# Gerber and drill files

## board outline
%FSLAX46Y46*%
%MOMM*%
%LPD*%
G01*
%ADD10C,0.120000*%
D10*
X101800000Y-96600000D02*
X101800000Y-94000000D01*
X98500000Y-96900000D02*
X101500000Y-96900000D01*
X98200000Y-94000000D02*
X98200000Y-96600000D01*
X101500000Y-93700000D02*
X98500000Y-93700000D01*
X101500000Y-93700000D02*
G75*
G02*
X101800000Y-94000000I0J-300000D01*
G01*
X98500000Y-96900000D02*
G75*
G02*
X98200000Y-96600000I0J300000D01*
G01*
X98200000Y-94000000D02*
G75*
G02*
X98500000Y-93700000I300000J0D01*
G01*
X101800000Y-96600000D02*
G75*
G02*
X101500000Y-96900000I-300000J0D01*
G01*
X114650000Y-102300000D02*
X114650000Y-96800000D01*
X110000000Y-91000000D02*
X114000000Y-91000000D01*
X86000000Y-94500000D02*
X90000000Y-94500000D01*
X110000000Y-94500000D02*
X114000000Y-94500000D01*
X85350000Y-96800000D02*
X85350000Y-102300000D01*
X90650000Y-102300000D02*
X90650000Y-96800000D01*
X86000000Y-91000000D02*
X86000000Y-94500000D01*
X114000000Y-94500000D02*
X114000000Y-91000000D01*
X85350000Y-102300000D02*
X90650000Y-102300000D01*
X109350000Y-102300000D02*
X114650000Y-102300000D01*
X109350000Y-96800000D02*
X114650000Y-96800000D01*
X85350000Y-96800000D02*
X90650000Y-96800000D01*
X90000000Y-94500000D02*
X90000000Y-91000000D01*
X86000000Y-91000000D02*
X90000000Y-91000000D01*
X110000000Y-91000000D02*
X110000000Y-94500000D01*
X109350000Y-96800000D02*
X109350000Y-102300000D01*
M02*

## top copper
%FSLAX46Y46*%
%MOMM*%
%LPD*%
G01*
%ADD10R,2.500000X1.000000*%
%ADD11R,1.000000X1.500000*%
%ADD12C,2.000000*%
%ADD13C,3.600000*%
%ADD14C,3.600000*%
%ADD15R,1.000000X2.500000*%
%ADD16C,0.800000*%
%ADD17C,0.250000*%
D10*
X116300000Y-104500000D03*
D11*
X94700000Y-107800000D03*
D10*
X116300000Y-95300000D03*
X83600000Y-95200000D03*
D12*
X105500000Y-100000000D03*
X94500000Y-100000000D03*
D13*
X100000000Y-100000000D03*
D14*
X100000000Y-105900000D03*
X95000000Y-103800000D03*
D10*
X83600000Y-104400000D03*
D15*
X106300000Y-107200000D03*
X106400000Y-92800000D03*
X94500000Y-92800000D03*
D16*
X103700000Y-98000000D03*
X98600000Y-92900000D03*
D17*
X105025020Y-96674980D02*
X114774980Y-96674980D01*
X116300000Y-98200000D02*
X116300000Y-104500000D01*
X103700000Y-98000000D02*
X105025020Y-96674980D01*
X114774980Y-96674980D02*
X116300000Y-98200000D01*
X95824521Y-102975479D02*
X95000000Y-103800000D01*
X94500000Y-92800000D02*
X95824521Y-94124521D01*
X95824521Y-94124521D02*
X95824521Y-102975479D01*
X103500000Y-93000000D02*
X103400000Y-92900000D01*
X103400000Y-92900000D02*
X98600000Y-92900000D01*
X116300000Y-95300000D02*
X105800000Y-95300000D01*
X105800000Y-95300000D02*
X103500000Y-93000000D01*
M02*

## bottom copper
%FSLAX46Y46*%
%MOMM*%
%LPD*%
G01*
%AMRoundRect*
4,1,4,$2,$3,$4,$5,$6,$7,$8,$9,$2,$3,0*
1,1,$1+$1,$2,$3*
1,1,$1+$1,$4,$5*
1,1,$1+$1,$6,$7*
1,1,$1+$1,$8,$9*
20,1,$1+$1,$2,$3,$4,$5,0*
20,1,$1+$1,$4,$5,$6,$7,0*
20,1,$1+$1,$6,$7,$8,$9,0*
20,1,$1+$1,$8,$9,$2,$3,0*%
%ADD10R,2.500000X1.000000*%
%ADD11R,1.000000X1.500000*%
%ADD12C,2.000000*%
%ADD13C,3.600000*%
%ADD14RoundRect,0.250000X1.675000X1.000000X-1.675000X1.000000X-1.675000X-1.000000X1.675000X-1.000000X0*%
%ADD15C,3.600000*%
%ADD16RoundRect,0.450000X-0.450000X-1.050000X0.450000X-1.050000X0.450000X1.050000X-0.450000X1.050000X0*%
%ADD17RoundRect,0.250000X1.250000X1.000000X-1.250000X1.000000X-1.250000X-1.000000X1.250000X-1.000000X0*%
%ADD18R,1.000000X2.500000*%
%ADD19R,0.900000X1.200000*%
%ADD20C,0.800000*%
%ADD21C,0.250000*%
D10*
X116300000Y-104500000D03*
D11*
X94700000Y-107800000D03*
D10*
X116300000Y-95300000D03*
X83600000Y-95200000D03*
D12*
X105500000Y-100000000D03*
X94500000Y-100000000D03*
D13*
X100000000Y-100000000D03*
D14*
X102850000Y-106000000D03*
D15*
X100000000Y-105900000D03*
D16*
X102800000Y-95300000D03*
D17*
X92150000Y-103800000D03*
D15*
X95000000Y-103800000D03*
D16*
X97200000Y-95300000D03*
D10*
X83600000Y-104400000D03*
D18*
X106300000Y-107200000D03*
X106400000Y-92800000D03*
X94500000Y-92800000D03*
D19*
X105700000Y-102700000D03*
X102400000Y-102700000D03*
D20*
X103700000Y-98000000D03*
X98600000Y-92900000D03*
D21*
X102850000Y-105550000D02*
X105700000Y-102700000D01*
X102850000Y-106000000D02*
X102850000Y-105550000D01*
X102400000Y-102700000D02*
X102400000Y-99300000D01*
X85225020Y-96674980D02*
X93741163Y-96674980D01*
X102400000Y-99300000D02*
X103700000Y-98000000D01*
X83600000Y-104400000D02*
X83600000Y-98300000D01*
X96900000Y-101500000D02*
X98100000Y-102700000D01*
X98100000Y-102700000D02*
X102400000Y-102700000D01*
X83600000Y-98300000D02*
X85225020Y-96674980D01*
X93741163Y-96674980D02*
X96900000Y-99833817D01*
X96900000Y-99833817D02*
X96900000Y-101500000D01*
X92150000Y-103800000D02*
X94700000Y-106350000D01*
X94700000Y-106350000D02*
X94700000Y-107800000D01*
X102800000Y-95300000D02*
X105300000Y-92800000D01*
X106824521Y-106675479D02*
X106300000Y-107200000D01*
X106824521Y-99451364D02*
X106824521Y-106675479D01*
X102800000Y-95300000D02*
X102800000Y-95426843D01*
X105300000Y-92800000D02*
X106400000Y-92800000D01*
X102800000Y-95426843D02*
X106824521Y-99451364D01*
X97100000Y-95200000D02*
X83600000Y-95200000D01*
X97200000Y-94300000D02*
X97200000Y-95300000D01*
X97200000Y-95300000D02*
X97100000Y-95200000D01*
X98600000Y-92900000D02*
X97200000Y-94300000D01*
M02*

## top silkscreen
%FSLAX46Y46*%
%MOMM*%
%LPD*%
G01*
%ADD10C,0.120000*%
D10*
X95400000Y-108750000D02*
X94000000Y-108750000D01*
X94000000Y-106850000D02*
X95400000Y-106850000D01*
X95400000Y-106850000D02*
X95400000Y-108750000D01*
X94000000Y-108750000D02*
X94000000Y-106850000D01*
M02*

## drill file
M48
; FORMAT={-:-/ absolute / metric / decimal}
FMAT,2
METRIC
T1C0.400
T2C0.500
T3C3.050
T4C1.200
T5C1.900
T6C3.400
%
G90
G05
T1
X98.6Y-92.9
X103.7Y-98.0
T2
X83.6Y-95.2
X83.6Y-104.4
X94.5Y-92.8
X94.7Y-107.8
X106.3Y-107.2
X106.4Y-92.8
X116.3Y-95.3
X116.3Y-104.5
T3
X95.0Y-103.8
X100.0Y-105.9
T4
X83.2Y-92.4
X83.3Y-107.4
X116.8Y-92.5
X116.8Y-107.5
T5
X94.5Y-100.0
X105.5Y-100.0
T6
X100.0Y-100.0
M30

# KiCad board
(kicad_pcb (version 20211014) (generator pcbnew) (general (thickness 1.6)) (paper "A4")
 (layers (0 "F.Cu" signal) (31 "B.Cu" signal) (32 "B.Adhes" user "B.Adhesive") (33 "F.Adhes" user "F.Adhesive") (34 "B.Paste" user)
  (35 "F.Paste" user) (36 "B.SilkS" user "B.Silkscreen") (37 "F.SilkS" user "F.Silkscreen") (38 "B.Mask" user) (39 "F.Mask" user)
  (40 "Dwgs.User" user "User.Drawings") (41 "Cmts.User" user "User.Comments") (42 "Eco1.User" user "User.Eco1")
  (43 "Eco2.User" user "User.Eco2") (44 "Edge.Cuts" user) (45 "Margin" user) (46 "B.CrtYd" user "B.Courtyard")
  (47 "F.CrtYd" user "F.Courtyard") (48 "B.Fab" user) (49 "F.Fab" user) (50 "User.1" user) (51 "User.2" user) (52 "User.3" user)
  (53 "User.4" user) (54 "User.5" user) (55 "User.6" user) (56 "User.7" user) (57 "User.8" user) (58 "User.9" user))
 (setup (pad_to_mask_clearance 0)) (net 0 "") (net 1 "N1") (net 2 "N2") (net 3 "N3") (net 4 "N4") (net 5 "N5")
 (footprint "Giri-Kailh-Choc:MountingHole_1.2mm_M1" (layer "F.Cu") (at 116.8 92.5)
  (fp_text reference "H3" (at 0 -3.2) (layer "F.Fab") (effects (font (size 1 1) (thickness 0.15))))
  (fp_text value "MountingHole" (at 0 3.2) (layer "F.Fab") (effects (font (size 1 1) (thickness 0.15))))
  (pad "" np_thru_hole circle (at 0 0) (size 1.2 1.2) (drill 1.2) (layers F&B.Cu *.Mask)))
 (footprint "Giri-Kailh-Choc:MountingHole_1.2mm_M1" (layer "F.Cu") (at 116.8 107.5)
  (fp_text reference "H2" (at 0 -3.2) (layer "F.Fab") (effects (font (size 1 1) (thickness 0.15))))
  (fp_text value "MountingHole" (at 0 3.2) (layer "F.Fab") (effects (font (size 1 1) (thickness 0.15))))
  (pad "" np_thru_hole circle (at 0 0) (size 1.2 1.2) (drill 1.2) (layers F&B.Cu *.Mask)))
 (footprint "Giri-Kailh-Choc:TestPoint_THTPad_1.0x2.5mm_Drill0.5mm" (layer "F.Cu") (at 116.3 104.5)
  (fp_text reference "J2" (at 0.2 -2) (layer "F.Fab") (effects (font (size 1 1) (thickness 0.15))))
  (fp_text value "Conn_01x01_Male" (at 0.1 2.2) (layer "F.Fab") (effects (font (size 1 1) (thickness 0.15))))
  (pad "1" thru_hole rect (at 0 0) (size 2.5 1) (drill 0.5) (layers *.Cu *.Mask) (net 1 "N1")))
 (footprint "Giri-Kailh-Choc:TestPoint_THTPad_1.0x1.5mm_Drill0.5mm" (layer "F.Cu") (at 94.7 107.8 90)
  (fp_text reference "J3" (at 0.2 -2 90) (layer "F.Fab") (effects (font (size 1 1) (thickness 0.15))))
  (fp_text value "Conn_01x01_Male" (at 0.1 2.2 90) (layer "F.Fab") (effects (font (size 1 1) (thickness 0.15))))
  (fp_line (start -0.95 0.7) (end -0.95 -0.7) (layer "F.SilkS") (width 0.12))
  (fp_line (start 0.95 -0.7) (end 0.95 0.7) (layer "F.SilkS") (width 0.12))
  (fp_line (start 0.95 0.7) (end -0.95 0.7) (layer "F.SilkS") (width 0.12))
  (fp_line (start -0.95 -0.7) (end 0.95 -0.7) (layer "F.SilkS") (width 0.12))
  (pad "1" thru_hole rect (at 0 0 90) (size 1.5 1) (drill 0.5) (layers *.Cu *.Mask) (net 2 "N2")))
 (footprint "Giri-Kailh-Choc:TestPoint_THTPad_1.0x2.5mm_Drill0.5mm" (layer "F.Cu") (at 116.3 95.3)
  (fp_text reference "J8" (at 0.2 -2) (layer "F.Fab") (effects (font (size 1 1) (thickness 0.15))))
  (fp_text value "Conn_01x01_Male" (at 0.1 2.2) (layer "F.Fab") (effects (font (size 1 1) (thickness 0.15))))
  (pad "1" thru_hole rect (at 0 0) (size 2.5 1) (drill 0.5) (layers *.Cu *.Mask) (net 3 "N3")))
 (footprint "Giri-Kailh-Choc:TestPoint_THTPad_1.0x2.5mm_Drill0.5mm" (layer "F.Cu") (at 83.6 95.2)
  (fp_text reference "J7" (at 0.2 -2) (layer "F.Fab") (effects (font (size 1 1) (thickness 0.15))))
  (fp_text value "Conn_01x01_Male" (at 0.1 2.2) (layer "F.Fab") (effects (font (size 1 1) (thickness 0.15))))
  (pad "1" thru_hole rect (at 0 0) (size 2.5 1) (drill 0.5) (layers *.Cu *.Mask) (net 3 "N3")))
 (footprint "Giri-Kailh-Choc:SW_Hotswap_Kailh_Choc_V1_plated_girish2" (layer "F.Cu") (at 100 100)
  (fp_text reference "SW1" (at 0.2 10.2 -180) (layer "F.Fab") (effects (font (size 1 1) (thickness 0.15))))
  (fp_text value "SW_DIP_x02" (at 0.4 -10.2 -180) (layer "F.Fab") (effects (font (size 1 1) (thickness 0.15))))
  (fp_line (start 1.8 -3.4) (end 1.8 -6) (layer "Edge.Cuts") (width 0.12))
  (fp_line (start -1.5 -3.1) (end 1.5 -3.1) (layer "Edge.Cuts") (width 0.12))
  (fp_line (start -1.8 -6) (end -1.8 -3.4) (layer "Edge.Cuts") (width 0.12))
  (fp_line (start 1.5 -6.3) (end -1.5 -6.3) (layer "Edge.Cuts") (width 0.12))
  (fp_arc (start 1.5 -6.3) (mid 1.712132 -6.212132) (end 1.8 -6) (layer "Edge.Cuts") (width 0.12))
  (fp_arc (start -1.5 -3.1) (mid -1.712132 -3.187868) (end -1.8 -3.4) (layer "Edge.Cuts") (width 0.12))
  (fp_arc (start -1.8 -6) (mid -1.712132 -6.212132) (end -1.5 -6.3) (layer "Edge.Cuts") (width 0.12))
  (fp_arc (start 1.8 -3.4) (mid 1.712132 -3.187868) (end 1.5 -3.1) (layer "Edge.Cuts") (width 0.12))
  (pad "" smd roundrect (at -8.5 3.8 180) (size 1.9 2.5) (layers "B.Paste" "B.Mask") (roundrect_rratio 0.1))
  (pad "" np_thru_hole circle (at 5.5 0 180) (size 2 2) (drill 1.9) (layers F&B.Cu *.Mask))
  (pad "" np_thru_hole circle (at -5.5 0 180) (size 2 2) (drill 1.9) (layers F&B.Cu *.Mask))
  (pad "" smd roundrect (at 3.5 6 180) (size 2.55 2.5) (layers "B.Paste" "B.Mask") (roundrect_rratio 0.1))
  (pad "" np_thru_hole circle (at 0 0 180) (size 3.6 3.6) (drill 3.4) (layers F&B.Cu *.Mask))
  (pad "1" smd roundrect (at 2.85 6 180) (size 3.85 2.5) (layers "B.Cu" "B.Paste" "B.Mask") (roundrect_rratio 0.1) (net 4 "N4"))
  (pad "1" thru_hole circle (at 0 5.9 180) (size 3.6 3.6) (drill 3.05) (layers *.Cu "B.Mask") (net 4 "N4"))
  (pad "2" smd roundrect (at 2.8 -4.7) (size 1.8 3) (layers "B.Cu" "B.Paste" "B.Mask") (roundrect_rratio 0.25) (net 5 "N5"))
  (pad "3" smd roundrect (at -7.85 3.8 180) (size 3 2.5) (layers "B.Cu" "B.Paste" "B.Mask") (roundrect_rratio 0.1) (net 2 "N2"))
  (pad "3" thru_hole circle (at -5 3.8 180) (size 3.6 3.6) (drill 3.05) (layers *.Cu "B.Mask") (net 2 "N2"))
  (pad "4" smd roundrect (at -2.8 -4.7) (size 1.8 3) (layers "B.Cu" "B.Paste" "B.Mask") (roundrect_rratio 0.25) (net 3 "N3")))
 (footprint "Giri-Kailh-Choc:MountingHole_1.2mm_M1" (layer "F.Cu") (at 83.3 107.4)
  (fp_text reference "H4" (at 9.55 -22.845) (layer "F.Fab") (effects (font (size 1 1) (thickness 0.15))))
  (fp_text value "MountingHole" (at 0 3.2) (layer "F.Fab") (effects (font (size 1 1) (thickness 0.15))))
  (pad "" np_thru_hole circle (at 0 0) (size 1.2 1.2) (drill 1.2) (layers F&B.Cu *.Mask)))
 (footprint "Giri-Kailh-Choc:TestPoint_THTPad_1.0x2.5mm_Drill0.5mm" (layer "F.Cu") (at 83.6 104.4)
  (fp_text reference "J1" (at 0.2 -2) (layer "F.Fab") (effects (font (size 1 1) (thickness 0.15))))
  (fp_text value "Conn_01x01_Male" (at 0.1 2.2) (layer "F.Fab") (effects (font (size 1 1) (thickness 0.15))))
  (pad "1" thru_hole rect (at 0 0) (size 2.5 1) (drill 0.5) (layers *.Cu *.Mask) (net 1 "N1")))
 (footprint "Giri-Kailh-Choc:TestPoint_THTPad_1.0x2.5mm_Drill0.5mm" (layer "F.Cu") (at 106.3 107.2 90)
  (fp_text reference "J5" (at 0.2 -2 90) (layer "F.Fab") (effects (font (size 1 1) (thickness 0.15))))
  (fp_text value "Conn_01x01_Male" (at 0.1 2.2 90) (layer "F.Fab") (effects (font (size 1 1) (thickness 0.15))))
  (pad "1" thru_hole rect (at 0 0 90) (size 2.5 1) (drill 0.5) (layers *.Cu *.Mask) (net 5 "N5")))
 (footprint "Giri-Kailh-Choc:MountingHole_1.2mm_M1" (layer "F.Cu") (at 83.2 92.4)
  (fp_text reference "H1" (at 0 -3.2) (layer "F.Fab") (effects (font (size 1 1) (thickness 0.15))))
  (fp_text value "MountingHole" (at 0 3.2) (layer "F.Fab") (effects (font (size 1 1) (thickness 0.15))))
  (pad "" np_thru_hole circle (at 0 0) (size 1.2 1.2) (drill 1.2) (layers F&B.Cu *.Mask)))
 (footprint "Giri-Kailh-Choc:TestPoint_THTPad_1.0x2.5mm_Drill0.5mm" (layer "F.Cu") (at 106.4 92.8 90)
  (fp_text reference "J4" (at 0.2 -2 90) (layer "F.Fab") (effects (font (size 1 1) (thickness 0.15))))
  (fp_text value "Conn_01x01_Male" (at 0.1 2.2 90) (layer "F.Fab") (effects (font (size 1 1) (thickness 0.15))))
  (pad "1" thru_hole rect (at 0 0 90) (size 2.5 1) (drill 0.5) (layers *.Cu *.Mask) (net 5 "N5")))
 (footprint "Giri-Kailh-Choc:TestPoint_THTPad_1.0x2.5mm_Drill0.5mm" (layer "F.Cu") (at 94.5 92.8 90)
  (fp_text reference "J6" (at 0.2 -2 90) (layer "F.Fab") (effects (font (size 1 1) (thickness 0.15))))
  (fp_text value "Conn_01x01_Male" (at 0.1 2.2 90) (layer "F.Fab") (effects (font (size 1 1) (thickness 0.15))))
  (pad "1" thru_hole rect (at 0 0 90) (size 2.5 1) (drill 0.5) (layers *.Cu *.Mask) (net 2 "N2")))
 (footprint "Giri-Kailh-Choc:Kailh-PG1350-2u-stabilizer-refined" (layer "F.Cu") (at 100 100)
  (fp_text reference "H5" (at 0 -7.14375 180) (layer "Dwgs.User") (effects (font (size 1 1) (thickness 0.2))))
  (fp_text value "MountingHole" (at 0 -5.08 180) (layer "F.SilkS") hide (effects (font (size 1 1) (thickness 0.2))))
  (fp_line (start 14.65 2.3) (end 14.65 -3.2) (layer "Edge.Cuts") (width 0.12))
  (fp_line (start 10 -9) (end 14 -9) (layer "Edge.Cuts") (width 0.12))
  (fp_line (start -14 -5.5) (end -10 -5.5) (layer "Edge.Cuts") (width 0.12))
  (fp_line (start 10 -5.5) (end 14 -5.5) (layer "Edge.Cuts") (width 0.12))
  (fp_line (start -14.65 -3.2) (end -14.65 2.3) (layer "Edge.Cuts") (width 0.12))
  (fp_line (start -9.35 2.3) (end -9.35 -3.2) (layer "Edge.Cuts") (width 0.12))
  (fp_line (start -14 -9) (end -14 -5.5) (layer "Edge.Cuts") (width 0.12))
  (fp_line (start 14 -5.5) (end 14 -9) (layer "Edge.Cuts") (width 0.12))
  (fp_line (start -14.65 2.3) (end -9.35 2.3) (layer "Edge.Cuts") (width 0.12))
  (fp_line (start 9.35 2.3) (end 14.65 2.3) (layer "Edge.Cuts") (width 0.12))
  (fp_line (start 9.35 -3.2) (end 14.65 -3.2) (layer "Edge.Cuts") (width 0.12))
  (fp_line (start -14.65 -3.2) (end -9.35 -3.2) (layer "Edge.Cuts") (width 0.12))
  (fp_line (start -10 -5.5) (end -10 -9) (layer "Edge.Cuts") (width 0.12))
  (fp_line (start -14 -9) (end -10 -9) (layer "Edge.Cuts") (width 0.12))
  (fp_line (start 10 -9) (end 10 -5.5) (layer "Edge.Cuts") (width 0.12))
  (fp_line (start 9.35 -3.2) (end 9.35 2.3) (layer "Edge.Cuts") (width 0.12)))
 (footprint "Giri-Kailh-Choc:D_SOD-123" (layer "B.Cu") (at 104.05 102.7 180)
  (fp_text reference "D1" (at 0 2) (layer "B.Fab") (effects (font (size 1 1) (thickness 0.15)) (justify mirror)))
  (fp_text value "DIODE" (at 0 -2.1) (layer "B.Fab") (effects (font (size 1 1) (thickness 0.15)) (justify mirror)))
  (pad "1" smd rect (at -1.65 0 180) (size 0.9 1.2) (layers "B.Cu" "B.Paste" "B.Mask") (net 4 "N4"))
  (pad "2" smd rect (at 1.65 0 180) (size 0.9 1.2) (layers "B.Cu" "B.Paste" "B.Mask") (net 1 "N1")))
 (segment (start 102.85 105.55) (end 105.7 102.7) (width 0.25) (layer "B.Cu") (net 4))
 (segment (start 102.85 106) (end 102.85 105.55) (width 0.25) (layer "B.Cu") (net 4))
 (segment (start 105.02502 96.67498) (end 114.77498 96.67498) (width 0.25) (layer "F.Cu") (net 1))
 (segment (start 116.3 98.2) (end 116.3 104.5) (width 0.25) (layer "F.Cu") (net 1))
 (segment (start 103.7 98) (end 105.02502 96.67498) (width 0.25) (layer "F.Cu") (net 1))
 (segment (start 114.77498 96.67498) (end 116.3 98.2) (width 0.25) (layer "F.Cu") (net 1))
 (via (at 103.7 98) (size 0.8) (drill 0.4) (layers "F.Cu" "B.Cu") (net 1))
 (segment (start 102.4 102.7) (end 102.4 99.3) (width 0.25) (layer "B.Cu") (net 1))
 (segment (start 85.22502 96.67498) (end 93.741163 96.67498) (width 0.25) (layer "B.Cu") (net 1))
 (segment (start 102.4 99.3) (end 103.7 98) (width 0.25) (layer "B.Cu") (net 1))
 (segment (start 83.6 104.4) (end 83.6 98.3) (width 0.25) (layer "B.Cu") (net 1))
 (segment (start 96.9 101.5) (end 98.1 102.7) (width 0.25) (layer "B.Cu") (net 1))
 (segment (start 98.1 102.7) (end 102.4 102.7) (width 0.25) (layer "B.Cu") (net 1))
 (segment (start 83.6 98.3) (end 85.22502 96.67498) (width 0.25) (layer "B.Cu") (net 1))
 (segment (start 93.741163 96.67498) (end 96.9 99.833817) (width 0.25) (layer "B.Cu") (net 1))
 (segment (start 96.9 99.833817) (end 96.9 101.5) (width 0.25) (layer "B.Cu") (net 1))
 (segment (start 95.824521 102.975479) (end 95 103.8) (width 0.25) (layer "F.Cu") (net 2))
 (segment (start 94.5 92.8) (end 95.824521 94.124521) (width 0.25) (layer "F.Cu") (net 2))
 (segment (start 95.824521 94.124521) (end 95.824521 102.975479) (width 0.25) (layer "F.Cu") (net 2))
 (segment (start 92.15 103.8) (end 94.7 106.35) (width 0.25) (layer "B.Cu") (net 2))
 (segment (start 94.7 106.35) (end 94.7 107.8) (width 0.25) (layer "B.Cu") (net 2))
 (segment (start 102.8 95.3) (end 105.3 92.8) (width 0.25) (layer "B.Cu") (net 5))
 (segment (start 106.824521 106.675479) (end 106.3 107.2) (width 0.25) (layer "B.Cu") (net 5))
 (segment (start 106.824521 99.451364) (end 106.824521 106.675479) (width 0.25) (layer "B.Cu") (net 5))
 (segment (start 102.8 95.3) (end 102.8 95.426843) (width 0.25) (layer "B.Cu") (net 5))
 (segment (start 105.3 92.8) (end 106.4 92.8) (width 0.25) (layer "B.Cu") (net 5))
 (segment (start 102.8 95.426843) (end 106.824521 99.451364) (width 0.25) (layer "B.Cu") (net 5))
 (segment (start 103.5 93) (end 103.4 92.9) (width 0.25) (layer "F.Cu") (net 3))
 (segment (start 103.4 92.9) (end 98.6 92.9) (width 0.25) (layer "F.Cu") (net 3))
 (segment (start 116.3 95.3) (end 105.8 95.3) (width 0.25) (layer "F.Cu") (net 3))
 (segment (start 105.8 95.3) (end 103.5 93) (width 0.25) (layer "F.Cu") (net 3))
 (via (at 98.6 92.9) (size 0.8) (drill 0.4) (layers "F.Cu" "B.Cu") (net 3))
 (segment (start 97.1 95.2) (end 83.6 95.2) (width 0.25) (layer "B.Cu") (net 3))
 (segment (start 97.2 94.3) (end 97.2 95.3) (width 0.25) (layer "B.Cu") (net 3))
 (segment (start 97.2 95.3) (end 97.1 95.2) (width 0.25) (layer "B.Cu") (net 3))
 (segment (start 98.6 92.9) (end 97.2 94.3) (width 0.25) (layer "B.Cu") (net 3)))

